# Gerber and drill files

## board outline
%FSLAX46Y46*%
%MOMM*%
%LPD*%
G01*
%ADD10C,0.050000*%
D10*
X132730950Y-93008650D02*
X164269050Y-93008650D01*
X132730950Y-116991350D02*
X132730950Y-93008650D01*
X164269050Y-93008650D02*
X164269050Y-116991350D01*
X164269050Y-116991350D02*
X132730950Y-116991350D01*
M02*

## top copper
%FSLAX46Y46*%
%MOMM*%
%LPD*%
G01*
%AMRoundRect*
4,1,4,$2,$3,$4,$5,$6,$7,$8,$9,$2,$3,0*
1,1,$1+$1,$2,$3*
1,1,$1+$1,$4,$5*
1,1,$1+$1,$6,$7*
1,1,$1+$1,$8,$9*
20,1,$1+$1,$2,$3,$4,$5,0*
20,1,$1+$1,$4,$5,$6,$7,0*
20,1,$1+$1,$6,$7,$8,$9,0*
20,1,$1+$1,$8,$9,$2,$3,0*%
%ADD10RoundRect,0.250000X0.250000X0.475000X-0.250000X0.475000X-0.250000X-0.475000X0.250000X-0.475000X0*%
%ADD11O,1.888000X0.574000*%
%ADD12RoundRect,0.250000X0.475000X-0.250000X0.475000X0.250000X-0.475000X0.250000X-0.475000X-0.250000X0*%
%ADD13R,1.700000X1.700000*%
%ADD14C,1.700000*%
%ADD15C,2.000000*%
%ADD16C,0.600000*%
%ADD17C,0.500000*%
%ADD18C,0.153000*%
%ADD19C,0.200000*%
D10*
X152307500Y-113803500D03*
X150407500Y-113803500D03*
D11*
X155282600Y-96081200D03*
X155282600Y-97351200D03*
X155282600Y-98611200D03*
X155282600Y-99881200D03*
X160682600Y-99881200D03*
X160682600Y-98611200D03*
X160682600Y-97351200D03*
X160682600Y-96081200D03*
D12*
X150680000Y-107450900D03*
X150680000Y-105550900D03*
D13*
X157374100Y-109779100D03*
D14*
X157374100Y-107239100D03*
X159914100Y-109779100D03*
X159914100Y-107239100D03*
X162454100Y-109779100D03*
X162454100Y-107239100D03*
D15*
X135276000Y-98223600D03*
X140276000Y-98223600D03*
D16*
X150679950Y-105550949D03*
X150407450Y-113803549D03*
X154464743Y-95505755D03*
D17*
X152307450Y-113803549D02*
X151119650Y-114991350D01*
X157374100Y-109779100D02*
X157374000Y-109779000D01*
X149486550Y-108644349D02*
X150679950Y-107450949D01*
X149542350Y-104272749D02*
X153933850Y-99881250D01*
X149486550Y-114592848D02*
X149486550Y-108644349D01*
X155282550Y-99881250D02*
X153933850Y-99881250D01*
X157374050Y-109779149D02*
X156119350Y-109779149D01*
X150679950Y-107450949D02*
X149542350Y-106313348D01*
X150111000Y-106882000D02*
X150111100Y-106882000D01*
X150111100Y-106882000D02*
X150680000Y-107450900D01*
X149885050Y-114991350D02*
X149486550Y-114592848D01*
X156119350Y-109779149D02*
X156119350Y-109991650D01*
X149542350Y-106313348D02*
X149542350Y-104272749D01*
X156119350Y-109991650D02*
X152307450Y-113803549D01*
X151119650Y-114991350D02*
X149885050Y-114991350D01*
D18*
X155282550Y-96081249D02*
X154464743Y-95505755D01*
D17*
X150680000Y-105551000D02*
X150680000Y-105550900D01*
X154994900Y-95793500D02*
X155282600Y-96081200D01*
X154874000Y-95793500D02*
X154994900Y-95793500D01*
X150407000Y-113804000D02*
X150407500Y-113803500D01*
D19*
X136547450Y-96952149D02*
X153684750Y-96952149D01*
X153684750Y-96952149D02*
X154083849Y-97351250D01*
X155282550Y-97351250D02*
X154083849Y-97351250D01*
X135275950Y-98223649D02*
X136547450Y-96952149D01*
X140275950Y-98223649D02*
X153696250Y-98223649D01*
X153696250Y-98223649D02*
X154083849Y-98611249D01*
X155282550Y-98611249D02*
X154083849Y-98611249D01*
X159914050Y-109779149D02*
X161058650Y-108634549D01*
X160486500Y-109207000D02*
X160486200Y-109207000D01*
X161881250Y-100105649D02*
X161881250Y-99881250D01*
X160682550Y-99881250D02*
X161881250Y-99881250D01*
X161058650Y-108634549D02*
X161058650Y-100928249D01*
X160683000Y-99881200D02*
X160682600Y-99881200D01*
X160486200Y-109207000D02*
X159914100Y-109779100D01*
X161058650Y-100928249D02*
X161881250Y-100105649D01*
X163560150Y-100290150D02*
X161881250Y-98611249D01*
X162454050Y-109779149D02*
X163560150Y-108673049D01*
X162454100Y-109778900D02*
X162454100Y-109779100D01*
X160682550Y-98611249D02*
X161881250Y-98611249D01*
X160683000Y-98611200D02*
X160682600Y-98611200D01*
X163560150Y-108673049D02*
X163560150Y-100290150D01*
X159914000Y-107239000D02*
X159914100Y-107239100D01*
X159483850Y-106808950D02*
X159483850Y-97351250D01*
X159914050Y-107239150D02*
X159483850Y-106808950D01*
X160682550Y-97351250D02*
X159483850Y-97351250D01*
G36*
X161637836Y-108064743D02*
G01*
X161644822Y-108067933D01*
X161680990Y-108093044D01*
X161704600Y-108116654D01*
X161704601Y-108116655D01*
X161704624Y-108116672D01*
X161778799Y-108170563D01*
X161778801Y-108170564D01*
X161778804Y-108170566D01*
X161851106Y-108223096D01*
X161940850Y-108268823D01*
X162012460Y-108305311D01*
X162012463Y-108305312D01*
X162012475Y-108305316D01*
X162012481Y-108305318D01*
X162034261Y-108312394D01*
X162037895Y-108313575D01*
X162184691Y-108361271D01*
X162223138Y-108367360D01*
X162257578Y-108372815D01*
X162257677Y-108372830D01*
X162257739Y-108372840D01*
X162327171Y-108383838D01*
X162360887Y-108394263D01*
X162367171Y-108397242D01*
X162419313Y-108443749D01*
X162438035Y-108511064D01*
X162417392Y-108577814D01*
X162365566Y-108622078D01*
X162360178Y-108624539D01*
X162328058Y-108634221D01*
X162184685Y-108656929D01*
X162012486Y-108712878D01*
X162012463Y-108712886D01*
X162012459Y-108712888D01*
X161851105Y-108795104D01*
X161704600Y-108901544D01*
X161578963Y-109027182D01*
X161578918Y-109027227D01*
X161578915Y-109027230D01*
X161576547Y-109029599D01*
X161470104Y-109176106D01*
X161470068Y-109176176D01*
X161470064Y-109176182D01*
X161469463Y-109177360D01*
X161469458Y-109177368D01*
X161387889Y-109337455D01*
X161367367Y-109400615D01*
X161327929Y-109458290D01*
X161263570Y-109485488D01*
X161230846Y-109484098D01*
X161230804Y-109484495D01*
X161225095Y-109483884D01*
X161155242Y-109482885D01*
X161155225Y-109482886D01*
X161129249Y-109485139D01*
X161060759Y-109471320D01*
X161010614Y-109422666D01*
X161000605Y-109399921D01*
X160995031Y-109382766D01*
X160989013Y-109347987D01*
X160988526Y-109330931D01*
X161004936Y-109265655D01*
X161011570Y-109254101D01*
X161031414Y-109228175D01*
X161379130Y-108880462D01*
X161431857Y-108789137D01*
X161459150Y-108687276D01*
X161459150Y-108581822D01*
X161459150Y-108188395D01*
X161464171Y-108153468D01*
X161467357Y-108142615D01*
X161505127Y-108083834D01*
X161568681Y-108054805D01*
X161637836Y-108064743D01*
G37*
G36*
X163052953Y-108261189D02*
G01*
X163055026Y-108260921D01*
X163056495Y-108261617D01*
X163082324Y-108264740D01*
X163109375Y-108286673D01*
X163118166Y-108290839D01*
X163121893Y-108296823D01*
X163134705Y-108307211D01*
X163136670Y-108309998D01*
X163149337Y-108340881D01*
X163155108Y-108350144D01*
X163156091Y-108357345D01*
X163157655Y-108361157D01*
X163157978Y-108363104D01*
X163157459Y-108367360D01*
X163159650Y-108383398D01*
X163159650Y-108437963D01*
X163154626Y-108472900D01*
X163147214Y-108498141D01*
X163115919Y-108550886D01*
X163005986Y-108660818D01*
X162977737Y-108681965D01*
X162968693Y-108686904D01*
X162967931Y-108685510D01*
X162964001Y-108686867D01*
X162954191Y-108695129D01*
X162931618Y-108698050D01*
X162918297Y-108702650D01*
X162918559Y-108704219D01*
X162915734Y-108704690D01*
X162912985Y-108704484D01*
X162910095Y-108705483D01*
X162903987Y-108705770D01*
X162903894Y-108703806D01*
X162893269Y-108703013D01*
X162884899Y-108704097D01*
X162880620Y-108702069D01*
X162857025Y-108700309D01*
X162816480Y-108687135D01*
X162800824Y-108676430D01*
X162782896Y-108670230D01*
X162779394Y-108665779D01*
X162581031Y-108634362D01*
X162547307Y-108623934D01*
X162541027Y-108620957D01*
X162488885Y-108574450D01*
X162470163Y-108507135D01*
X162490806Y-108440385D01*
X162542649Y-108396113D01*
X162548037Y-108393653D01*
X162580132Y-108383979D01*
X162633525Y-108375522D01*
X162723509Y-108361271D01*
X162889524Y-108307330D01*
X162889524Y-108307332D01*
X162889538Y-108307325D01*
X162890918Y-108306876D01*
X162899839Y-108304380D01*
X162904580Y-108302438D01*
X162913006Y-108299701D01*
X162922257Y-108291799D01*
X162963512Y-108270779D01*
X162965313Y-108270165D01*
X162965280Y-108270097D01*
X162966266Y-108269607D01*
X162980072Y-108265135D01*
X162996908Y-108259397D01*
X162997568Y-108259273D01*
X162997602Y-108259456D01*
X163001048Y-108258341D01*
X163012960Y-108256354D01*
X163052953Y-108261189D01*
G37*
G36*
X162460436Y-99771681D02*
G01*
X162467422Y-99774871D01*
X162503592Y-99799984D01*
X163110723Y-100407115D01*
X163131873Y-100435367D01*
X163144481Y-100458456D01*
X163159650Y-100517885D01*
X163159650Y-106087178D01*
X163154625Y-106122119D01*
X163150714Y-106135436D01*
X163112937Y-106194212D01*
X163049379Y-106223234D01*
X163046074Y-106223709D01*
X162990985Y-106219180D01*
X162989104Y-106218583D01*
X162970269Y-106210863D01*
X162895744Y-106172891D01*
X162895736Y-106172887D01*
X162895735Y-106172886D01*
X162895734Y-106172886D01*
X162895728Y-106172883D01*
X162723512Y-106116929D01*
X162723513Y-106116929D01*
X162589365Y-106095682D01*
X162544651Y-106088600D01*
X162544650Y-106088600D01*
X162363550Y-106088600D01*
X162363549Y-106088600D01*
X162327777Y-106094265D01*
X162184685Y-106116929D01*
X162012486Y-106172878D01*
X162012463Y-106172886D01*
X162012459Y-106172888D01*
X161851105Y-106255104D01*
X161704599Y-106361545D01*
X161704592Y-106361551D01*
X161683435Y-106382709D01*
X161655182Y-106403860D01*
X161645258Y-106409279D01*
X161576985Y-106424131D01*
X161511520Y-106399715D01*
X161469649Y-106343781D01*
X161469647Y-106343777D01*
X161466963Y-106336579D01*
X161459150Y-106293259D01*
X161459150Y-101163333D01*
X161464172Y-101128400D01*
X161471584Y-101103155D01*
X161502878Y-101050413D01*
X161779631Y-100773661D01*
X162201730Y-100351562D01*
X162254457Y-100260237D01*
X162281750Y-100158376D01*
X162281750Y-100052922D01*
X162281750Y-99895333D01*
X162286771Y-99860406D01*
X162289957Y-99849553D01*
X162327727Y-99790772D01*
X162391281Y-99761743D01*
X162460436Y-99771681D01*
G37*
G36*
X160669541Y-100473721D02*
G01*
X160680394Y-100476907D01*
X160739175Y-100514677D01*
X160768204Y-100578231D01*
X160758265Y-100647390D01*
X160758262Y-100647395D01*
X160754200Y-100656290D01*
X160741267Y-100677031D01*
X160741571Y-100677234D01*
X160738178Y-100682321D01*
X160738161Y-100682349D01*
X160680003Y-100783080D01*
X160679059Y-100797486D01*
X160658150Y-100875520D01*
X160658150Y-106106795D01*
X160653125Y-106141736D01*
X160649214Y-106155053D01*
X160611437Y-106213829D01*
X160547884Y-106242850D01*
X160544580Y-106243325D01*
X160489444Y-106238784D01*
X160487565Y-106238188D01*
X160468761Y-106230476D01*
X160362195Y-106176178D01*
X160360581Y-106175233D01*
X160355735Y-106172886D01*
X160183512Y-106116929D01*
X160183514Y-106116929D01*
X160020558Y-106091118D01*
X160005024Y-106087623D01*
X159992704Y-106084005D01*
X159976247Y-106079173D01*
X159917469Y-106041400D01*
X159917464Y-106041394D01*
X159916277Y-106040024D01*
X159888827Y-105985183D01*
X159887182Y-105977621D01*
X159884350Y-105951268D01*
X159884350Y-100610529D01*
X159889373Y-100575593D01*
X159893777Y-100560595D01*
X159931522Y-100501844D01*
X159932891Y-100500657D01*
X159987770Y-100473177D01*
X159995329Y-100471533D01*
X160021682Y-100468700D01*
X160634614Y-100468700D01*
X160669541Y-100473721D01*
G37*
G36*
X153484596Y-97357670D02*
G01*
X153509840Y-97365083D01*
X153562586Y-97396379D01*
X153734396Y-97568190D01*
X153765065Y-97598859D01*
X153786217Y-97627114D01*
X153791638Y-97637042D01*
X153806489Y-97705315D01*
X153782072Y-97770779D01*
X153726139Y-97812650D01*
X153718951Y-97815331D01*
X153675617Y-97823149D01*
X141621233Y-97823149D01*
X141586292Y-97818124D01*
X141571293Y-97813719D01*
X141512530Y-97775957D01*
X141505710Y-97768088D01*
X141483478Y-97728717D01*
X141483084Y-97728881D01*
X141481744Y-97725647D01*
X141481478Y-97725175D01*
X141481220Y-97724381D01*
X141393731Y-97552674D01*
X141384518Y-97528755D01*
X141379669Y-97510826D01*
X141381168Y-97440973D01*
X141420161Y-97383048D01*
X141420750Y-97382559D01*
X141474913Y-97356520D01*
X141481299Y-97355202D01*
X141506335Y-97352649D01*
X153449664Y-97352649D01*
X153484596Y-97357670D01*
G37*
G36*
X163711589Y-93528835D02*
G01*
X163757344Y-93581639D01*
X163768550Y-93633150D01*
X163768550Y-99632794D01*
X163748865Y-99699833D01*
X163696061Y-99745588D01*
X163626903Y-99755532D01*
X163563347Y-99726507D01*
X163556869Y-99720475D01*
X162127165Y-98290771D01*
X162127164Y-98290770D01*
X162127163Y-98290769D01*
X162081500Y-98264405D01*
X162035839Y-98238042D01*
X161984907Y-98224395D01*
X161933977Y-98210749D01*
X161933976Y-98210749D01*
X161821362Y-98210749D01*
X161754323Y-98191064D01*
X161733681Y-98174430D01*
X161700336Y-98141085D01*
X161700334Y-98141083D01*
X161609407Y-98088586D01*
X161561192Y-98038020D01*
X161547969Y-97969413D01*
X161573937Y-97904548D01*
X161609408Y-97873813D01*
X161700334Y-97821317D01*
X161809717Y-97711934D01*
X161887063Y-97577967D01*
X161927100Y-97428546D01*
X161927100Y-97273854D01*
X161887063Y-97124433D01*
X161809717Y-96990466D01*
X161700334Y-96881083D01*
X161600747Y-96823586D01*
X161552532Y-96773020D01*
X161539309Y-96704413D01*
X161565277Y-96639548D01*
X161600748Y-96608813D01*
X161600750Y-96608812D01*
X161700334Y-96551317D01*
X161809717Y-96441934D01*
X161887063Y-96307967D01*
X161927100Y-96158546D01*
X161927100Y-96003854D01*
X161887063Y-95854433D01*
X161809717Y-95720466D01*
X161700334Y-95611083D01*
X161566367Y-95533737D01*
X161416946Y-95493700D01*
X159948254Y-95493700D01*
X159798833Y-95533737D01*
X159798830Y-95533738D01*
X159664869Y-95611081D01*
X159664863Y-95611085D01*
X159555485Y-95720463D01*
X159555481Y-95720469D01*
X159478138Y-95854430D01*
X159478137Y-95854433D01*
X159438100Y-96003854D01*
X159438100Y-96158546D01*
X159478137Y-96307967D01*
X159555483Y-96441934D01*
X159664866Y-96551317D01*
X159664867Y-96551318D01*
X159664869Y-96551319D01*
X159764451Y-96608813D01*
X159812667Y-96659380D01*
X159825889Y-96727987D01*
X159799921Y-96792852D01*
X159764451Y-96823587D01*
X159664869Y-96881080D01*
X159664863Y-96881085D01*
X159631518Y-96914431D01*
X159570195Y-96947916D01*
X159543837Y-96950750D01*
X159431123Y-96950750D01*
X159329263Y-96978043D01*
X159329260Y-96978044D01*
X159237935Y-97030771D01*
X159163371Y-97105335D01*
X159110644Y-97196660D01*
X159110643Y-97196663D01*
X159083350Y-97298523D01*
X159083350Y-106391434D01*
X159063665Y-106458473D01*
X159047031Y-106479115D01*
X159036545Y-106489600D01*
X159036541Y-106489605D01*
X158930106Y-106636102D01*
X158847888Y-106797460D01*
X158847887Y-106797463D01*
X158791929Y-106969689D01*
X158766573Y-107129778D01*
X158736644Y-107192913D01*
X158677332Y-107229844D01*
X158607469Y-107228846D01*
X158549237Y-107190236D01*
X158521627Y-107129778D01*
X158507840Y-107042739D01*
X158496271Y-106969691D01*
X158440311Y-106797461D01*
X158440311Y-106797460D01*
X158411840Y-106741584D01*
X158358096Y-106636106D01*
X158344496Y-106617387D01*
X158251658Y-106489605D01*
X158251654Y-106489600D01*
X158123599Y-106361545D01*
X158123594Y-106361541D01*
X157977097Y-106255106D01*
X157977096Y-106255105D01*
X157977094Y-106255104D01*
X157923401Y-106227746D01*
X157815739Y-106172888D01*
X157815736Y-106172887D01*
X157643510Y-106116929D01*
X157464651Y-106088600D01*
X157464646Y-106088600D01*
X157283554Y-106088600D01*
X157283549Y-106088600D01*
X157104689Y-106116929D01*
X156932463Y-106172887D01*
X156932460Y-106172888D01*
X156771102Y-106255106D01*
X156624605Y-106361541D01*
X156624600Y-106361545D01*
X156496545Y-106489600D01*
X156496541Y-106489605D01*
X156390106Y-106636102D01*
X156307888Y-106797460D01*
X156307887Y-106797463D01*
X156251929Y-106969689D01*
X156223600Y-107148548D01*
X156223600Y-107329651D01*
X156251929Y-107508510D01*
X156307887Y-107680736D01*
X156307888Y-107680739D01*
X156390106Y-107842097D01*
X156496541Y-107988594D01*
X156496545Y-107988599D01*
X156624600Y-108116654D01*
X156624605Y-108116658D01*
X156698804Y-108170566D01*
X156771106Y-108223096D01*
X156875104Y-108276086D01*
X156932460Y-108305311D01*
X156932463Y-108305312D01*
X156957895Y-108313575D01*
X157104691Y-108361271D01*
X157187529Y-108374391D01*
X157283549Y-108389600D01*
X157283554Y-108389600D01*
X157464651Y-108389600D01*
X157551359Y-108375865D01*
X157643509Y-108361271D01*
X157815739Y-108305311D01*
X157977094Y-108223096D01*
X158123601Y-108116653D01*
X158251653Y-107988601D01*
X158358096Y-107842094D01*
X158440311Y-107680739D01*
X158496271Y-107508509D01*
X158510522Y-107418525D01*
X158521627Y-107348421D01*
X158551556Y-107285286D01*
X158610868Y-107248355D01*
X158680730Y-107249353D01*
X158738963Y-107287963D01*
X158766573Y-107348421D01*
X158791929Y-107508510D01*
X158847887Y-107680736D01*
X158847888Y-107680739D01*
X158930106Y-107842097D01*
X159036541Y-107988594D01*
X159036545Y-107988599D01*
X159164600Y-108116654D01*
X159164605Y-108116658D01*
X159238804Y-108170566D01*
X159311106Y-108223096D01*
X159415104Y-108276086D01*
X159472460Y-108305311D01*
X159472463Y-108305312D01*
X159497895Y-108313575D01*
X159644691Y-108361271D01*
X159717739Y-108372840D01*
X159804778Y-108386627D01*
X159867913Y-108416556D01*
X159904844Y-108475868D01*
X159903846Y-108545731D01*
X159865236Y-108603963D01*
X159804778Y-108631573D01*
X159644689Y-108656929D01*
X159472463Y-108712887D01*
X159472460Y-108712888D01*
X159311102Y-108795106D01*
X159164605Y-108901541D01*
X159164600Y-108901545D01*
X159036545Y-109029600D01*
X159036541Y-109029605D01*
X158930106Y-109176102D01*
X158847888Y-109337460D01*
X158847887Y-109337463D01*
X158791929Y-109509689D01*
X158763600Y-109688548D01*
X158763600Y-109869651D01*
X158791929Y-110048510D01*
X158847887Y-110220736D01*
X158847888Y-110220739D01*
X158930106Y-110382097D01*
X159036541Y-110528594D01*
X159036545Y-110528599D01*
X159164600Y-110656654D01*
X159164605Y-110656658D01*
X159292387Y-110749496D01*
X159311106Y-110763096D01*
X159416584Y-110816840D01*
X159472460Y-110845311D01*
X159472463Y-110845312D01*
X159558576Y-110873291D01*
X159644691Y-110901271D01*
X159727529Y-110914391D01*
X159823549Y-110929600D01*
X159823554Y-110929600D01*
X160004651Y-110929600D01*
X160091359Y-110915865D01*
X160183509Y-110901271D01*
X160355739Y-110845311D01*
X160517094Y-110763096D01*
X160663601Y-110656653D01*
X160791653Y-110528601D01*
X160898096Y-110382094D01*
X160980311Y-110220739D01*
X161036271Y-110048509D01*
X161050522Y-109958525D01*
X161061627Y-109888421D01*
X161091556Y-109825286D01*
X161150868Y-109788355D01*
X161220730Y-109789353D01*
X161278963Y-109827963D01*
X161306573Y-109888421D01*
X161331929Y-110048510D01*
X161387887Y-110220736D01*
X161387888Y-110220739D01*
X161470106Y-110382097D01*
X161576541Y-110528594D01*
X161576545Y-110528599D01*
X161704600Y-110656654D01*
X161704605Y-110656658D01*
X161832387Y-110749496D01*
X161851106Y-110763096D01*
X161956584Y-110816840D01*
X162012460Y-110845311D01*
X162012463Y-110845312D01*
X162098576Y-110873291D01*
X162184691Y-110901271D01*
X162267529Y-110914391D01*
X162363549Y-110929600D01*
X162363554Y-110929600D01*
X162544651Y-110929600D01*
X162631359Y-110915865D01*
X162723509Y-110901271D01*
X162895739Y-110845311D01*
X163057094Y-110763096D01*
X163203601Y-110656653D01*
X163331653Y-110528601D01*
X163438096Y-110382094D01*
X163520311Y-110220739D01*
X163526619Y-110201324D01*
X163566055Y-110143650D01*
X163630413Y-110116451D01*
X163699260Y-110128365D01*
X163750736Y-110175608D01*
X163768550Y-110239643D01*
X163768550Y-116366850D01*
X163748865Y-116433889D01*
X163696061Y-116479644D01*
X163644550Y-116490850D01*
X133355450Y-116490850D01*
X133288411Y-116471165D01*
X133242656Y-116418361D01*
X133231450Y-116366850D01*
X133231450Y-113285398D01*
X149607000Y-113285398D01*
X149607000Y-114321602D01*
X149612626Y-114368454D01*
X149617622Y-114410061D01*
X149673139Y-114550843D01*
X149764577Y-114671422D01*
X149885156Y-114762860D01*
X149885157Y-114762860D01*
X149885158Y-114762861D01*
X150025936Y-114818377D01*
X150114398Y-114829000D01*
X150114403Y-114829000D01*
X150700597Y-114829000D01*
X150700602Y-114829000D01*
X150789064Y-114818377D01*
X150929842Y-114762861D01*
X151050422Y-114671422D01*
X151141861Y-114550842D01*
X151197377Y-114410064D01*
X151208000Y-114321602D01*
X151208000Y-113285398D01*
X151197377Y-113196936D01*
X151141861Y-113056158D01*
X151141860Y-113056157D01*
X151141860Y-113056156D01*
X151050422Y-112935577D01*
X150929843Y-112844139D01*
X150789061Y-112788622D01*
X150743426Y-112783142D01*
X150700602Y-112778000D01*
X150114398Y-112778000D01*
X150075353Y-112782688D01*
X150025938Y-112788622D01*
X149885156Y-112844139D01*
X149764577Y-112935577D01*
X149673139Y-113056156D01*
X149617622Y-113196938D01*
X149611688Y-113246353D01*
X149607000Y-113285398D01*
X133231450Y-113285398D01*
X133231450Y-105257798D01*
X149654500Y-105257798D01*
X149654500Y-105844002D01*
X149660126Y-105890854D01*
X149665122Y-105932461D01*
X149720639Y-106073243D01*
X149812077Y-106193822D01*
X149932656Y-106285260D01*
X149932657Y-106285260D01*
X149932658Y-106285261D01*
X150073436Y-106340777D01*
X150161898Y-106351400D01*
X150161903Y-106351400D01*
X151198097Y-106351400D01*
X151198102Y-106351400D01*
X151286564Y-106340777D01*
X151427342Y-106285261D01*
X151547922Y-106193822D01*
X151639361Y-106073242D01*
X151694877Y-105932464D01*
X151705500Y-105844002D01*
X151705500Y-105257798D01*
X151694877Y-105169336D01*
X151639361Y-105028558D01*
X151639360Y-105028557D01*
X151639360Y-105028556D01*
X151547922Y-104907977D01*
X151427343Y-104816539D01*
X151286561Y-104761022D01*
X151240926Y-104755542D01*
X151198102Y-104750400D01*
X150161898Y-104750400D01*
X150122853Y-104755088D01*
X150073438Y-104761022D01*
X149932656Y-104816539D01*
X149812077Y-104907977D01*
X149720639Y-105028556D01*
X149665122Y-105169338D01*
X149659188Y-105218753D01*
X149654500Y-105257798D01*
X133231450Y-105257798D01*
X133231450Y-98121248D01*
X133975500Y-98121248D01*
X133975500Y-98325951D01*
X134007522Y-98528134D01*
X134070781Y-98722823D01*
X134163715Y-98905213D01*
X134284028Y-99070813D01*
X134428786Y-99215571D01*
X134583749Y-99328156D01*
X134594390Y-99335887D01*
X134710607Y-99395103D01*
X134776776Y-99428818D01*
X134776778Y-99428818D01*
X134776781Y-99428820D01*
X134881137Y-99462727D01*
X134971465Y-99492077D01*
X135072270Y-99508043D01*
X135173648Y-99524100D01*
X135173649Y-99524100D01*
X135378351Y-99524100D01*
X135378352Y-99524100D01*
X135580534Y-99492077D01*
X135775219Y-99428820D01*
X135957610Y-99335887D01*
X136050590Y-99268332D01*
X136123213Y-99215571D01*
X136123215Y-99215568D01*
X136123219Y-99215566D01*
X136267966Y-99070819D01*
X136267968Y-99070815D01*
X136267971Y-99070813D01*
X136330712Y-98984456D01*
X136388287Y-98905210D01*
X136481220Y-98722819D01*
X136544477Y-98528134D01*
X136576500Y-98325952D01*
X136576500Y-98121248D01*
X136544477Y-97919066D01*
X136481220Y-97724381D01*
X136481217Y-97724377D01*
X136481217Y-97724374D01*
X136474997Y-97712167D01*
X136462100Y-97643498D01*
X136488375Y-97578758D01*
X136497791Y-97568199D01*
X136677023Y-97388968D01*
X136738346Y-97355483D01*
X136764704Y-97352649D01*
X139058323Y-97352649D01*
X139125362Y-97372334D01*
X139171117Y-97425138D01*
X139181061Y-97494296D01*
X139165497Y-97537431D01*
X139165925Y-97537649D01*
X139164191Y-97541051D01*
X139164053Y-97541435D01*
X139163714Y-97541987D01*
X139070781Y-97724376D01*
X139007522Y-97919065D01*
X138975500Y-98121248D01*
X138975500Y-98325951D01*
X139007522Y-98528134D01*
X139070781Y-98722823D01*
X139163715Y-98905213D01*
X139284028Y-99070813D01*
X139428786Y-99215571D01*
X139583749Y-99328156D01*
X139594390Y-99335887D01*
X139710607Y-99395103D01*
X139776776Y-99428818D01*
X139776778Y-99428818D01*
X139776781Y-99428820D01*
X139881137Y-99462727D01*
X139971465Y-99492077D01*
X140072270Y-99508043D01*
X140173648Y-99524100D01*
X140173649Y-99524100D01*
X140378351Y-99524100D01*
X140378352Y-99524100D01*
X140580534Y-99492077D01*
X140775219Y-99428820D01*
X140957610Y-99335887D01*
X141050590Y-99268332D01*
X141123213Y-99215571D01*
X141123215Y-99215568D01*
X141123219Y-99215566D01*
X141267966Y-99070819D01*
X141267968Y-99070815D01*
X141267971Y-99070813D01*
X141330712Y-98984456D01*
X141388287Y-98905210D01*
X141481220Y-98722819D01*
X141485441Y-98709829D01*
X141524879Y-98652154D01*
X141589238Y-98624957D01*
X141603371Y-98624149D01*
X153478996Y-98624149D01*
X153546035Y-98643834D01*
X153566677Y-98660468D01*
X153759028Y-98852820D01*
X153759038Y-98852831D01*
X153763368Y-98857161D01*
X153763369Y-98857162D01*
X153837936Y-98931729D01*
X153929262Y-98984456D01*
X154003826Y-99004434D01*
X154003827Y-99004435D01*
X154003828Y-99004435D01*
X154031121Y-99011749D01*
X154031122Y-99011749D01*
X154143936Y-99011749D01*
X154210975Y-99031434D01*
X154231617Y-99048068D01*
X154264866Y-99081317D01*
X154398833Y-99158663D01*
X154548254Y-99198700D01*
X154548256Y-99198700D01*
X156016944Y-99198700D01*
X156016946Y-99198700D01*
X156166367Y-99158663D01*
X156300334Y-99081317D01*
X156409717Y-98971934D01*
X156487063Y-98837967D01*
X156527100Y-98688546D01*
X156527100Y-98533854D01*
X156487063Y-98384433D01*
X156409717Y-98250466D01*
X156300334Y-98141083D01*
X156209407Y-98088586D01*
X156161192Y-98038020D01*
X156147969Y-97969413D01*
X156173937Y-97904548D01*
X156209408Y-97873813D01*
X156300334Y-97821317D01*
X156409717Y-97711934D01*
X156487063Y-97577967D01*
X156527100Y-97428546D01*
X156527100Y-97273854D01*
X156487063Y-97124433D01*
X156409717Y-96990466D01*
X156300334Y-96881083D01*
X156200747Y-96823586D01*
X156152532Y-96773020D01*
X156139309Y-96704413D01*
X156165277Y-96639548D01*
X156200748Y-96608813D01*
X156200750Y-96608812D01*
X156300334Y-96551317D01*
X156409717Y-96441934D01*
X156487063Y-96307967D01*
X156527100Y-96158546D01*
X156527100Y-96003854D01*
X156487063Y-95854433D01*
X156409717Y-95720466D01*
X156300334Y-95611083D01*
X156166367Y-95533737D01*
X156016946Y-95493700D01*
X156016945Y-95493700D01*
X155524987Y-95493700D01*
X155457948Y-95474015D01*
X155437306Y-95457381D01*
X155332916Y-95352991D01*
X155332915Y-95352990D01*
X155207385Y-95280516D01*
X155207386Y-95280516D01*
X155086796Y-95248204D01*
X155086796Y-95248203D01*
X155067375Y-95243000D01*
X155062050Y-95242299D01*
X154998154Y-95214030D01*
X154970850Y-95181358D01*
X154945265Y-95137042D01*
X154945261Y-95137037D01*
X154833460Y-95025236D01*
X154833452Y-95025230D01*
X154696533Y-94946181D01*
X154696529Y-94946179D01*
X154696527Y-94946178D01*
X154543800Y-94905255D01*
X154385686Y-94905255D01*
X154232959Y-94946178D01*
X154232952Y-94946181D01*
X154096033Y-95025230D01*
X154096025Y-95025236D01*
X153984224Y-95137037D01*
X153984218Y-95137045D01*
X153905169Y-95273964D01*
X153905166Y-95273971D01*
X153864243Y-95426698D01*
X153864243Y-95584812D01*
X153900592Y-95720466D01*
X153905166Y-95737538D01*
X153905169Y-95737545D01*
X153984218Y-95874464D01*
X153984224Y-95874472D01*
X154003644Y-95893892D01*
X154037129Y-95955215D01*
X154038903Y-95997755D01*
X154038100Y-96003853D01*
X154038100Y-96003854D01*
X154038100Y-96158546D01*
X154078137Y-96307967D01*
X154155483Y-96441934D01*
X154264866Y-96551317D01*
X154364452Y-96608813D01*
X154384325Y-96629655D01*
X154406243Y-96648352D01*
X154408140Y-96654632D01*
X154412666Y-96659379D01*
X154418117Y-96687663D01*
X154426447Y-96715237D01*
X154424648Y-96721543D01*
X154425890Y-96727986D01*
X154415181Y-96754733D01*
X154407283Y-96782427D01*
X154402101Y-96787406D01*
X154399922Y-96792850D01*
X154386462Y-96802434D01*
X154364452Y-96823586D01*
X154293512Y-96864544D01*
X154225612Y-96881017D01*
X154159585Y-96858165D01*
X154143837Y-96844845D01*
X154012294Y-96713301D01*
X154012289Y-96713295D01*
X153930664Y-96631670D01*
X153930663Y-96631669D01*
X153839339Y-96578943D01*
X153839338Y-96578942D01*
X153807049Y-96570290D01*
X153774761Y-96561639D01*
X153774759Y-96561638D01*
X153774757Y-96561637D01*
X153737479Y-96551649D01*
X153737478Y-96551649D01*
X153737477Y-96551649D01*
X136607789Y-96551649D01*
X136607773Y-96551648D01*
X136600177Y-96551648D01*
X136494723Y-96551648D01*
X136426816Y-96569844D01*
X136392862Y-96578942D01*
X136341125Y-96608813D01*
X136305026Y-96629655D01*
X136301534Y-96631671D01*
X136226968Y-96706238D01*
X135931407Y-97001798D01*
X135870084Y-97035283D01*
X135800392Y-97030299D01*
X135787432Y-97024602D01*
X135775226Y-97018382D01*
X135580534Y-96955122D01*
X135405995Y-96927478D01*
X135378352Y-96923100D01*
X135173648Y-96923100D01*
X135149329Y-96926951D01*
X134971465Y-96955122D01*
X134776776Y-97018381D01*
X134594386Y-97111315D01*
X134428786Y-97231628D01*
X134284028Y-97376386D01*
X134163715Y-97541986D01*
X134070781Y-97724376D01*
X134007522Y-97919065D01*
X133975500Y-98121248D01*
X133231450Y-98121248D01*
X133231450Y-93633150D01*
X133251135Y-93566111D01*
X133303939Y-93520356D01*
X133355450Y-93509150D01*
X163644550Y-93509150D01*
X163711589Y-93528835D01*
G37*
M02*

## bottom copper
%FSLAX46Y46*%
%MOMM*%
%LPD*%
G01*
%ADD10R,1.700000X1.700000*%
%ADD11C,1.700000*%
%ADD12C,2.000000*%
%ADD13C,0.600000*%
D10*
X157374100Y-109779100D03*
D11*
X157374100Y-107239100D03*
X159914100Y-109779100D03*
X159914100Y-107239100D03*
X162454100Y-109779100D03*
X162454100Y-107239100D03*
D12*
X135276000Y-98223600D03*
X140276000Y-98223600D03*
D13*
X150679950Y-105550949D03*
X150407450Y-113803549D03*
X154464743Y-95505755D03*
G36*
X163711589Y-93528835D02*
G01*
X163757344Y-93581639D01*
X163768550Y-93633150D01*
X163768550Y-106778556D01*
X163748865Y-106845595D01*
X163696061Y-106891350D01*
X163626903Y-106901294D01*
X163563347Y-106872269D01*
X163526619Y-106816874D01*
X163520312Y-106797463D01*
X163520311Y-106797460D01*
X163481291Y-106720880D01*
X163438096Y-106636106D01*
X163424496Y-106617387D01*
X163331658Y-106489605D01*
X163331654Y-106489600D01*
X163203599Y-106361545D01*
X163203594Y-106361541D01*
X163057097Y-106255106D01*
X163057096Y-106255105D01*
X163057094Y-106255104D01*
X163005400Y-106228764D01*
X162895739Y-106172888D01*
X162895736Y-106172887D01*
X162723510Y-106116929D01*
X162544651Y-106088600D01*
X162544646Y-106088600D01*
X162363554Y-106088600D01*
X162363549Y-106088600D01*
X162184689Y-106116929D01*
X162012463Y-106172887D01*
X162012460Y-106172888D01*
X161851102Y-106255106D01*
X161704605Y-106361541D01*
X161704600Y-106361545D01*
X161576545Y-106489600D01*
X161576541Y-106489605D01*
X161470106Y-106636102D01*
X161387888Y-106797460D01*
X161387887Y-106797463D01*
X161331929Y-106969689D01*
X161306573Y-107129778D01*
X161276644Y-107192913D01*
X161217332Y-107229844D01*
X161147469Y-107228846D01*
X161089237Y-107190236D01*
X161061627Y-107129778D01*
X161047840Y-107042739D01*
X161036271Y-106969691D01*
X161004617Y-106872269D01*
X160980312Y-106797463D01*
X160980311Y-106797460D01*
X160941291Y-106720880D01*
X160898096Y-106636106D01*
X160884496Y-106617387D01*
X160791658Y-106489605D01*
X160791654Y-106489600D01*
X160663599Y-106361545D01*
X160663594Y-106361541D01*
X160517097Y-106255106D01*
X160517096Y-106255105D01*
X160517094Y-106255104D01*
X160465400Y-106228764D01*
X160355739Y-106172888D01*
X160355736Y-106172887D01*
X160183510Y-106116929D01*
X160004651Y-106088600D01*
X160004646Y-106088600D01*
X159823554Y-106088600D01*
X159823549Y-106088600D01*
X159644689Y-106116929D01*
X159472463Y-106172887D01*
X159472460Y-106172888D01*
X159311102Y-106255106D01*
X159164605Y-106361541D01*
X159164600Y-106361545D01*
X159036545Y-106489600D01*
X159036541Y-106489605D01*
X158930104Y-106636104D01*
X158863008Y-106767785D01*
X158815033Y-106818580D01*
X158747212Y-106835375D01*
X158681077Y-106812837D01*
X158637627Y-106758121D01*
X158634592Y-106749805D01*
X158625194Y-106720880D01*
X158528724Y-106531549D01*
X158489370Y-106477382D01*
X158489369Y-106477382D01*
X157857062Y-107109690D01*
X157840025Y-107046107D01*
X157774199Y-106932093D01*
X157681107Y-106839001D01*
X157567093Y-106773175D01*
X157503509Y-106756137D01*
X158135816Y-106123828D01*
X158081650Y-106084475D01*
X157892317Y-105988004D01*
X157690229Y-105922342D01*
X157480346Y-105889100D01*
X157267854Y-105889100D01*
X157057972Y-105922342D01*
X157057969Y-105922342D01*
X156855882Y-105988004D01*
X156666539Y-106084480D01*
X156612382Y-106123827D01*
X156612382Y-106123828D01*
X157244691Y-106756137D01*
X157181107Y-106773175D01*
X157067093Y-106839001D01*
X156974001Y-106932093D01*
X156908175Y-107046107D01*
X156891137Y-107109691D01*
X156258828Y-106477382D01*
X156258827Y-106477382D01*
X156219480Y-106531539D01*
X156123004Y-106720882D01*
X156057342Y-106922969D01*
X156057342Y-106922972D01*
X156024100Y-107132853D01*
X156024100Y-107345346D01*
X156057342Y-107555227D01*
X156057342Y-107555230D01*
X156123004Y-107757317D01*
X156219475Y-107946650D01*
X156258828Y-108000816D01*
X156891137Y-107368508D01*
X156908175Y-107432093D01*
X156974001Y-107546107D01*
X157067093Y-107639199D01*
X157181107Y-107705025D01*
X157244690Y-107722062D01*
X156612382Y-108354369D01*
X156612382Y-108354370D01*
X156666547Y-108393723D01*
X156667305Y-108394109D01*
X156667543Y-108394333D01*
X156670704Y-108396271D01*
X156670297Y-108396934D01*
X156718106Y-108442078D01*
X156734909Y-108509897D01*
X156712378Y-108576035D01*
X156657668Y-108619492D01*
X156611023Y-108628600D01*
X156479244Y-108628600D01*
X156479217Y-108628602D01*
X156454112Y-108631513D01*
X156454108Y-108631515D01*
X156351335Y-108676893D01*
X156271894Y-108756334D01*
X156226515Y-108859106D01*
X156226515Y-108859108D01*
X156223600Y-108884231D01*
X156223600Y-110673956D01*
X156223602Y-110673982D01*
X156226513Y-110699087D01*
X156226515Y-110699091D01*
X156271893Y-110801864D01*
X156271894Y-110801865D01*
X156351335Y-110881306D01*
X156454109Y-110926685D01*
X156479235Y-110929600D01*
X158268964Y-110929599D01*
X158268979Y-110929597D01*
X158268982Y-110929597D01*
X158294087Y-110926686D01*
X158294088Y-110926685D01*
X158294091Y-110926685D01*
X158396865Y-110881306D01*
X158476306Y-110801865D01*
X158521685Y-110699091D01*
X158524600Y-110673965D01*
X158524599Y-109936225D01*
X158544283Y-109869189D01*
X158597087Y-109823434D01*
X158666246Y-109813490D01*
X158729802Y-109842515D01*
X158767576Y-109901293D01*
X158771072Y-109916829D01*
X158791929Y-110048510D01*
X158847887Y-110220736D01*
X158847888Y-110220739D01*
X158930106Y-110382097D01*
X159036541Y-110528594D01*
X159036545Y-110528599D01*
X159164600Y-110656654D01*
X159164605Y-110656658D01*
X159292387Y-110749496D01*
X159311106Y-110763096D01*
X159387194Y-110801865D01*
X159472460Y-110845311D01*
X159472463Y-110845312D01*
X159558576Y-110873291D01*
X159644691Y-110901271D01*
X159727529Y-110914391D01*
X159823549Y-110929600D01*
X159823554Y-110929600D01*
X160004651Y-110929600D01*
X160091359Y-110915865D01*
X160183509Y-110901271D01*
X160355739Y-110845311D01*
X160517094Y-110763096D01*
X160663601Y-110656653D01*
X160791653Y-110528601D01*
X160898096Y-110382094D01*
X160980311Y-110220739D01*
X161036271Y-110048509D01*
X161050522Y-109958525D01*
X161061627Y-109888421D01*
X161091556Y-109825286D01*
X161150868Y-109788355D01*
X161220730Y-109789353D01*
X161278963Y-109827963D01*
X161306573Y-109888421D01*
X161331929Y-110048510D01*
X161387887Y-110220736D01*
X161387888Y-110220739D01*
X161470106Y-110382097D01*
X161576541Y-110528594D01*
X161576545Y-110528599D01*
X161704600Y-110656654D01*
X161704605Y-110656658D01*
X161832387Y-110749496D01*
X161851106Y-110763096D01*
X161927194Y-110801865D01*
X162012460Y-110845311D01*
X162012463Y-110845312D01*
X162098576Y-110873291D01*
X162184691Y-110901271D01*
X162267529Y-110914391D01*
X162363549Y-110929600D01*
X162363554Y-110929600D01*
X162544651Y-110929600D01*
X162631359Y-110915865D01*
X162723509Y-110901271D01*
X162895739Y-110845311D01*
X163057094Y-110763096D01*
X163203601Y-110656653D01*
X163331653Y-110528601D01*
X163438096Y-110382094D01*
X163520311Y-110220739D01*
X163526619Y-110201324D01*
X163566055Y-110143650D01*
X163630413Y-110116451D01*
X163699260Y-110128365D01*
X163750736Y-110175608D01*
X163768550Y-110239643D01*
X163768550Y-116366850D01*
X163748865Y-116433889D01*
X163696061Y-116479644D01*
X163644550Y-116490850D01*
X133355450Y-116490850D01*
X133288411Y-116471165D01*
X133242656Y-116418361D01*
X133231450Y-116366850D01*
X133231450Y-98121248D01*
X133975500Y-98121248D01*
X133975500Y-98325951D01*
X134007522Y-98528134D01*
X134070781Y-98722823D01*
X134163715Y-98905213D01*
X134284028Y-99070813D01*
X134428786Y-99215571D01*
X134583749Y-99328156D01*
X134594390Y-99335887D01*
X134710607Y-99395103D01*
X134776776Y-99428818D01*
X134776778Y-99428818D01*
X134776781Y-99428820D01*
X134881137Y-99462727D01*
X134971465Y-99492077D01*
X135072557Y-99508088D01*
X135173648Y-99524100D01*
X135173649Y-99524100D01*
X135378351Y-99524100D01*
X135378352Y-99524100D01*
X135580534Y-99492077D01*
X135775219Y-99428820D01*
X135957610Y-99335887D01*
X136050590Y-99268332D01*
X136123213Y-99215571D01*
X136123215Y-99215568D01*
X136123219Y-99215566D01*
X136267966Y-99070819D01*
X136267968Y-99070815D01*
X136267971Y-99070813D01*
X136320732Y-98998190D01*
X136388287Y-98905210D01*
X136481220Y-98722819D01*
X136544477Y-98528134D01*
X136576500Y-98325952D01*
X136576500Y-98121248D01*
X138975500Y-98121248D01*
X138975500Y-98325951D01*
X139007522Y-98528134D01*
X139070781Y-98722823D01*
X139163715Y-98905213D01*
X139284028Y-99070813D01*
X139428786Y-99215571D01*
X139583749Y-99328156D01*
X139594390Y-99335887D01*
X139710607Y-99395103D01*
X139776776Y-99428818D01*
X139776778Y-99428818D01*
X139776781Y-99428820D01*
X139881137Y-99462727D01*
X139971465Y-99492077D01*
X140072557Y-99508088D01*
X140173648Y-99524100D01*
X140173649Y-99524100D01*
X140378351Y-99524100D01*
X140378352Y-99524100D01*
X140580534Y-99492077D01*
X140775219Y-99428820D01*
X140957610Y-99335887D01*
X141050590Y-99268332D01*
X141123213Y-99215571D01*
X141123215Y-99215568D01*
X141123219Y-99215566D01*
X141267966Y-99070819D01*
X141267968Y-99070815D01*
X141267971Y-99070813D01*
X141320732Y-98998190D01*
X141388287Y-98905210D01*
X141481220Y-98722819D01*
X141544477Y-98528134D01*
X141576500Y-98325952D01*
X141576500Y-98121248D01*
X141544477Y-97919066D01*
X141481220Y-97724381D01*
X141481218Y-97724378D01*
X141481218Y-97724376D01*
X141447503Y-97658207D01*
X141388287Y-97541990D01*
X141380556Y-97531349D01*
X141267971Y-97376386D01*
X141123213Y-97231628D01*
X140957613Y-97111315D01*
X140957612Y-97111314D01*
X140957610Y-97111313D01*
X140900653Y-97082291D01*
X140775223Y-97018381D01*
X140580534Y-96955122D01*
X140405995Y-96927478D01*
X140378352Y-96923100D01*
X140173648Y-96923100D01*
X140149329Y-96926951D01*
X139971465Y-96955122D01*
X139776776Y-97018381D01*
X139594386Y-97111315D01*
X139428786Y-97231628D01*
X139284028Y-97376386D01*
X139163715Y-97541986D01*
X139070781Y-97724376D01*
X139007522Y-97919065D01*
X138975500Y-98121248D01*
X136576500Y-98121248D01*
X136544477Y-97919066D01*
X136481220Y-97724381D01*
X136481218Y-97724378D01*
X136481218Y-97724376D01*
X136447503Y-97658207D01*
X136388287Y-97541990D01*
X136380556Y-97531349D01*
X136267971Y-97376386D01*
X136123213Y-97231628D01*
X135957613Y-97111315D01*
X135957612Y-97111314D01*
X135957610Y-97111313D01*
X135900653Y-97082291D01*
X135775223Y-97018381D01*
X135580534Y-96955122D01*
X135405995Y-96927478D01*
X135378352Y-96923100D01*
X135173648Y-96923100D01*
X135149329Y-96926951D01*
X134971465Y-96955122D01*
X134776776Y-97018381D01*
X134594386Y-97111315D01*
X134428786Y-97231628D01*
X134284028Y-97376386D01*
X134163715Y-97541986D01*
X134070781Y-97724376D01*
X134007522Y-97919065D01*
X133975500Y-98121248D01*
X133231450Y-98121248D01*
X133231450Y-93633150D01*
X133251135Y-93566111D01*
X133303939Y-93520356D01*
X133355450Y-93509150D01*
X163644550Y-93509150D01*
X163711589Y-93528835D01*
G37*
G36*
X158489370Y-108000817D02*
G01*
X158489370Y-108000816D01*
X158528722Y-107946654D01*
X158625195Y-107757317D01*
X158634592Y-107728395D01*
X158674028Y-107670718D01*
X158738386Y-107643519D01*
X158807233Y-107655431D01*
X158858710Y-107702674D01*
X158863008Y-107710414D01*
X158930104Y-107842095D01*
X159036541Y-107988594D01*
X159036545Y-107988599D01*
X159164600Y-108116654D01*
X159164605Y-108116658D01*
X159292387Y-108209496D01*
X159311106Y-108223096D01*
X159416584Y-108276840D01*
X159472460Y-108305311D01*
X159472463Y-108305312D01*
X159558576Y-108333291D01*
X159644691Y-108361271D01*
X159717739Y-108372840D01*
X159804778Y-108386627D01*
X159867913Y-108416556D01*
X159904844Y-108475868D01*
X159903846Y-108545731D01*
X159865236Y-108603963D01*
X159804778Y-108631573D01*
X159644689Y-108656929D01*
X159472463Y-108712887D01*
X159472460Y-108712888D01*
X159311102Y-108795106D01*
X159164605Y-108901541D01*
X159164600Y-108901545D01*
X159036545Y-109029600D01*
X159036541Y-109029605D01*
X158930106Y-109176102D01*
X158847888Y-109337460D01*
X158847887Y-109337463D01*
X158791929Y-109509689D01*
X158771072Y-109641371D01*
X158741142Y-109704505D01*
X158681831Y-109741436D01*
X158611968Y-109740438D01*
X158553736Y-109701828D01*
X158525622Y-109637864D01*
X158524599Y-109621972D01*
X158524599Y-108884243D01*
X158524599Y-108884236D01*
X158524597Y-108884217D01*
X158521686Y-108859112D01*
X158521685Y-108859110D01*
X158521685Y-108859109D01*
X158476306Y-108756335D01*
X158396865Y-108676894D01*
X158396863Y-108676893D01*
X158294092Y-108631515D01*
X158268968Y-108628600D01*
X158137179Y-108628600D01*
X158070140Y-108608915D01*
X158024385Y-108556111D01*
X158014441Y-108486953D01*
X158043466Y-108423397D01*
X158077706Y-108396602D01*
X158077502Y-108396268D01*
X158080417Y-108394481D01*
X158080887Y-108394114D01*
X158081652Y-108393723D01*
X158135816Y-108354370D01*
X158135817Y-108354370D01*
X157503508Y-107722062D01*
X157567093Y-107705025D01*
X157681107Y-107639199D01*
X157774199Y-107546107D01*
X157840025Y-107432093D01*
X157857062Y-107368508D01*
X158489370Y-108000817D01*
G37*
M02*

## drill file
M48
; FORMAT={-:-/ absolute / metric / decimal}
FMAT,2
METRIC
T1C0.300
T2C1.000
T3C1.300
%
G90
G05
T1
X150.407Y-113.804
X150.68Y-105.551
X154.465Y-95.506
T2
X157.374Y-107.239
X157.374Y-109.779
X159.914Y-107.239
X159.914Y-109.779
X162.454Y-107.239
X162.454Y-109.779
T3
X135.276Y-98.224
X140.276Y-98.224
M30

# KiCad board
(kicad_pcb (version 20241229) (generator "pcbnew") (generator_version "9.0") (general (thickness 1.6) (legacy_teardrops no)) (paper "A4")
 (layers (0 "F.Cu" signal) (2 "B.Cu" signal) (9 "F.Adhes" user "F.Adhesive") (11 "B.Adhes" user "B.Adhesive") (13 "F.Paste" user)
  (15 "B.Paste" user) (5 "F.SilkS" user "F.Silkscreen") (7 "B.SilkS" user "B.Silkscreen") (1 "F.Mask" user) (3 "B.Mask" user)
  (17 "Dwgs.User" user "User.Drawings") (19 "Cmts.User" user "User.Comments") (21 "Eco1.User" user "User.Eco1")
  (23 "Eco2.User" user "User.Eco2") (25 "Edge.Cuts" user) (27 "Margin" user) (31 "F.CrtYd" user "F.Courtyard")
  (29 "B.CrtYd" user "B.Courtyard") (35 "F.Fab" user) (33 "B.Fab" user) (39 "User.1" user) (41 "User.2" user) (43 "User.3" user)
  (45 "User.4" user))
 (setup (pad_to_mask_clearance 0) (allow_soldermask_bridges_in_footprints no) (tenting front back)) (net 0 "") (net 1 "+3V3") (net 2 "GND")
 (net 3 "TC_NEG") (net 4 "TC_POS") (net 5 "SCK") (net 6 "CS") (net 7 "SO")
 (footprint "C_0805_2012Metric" (layer "F.Cu") (at 151.3575 113.8035 180)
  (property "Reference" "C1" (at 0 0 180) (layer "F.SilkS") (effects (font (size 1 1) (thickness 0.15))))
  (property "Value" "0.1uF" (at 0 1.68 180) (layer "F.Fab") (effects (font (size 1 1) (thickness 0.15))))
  (pad "1" smd roundrect (at -0.95 0 180) (size 1 1.45) (layers "F.Cu" "F.Mask" "F.Paste") (roundrect_rratio 0.25) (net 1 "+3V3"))
  (pad "2" smd roundrect (at 0.95 0 180) (size 1 1.45) (layers "F.Cu" "F.Mask" "F.Paste") (roundrect_rratio 0.25) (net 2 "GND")))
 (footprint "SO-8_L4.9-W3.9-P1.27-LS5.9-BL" (layer "F.Cu") (at 157.9826 97.9812 -90)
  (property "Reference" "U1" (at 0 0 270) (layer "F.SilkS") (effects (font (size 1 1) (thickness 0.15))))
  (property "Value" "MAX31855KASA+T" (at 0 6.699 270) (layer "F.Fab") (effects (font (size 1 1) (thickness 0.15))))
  (pad "1" smd oval (at -1.9 2.7 270) (size 0.574 1.888) (layers "F.Cu" "F.Mask" "F.Paste") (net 2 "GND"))
  (pad "2" smd oval (at -0.63 2.7 270) (size 0.574 1.888) (layers "F.Cu" "F.Mask" "F.Paste") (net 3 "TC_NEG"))
  (pad "3" smd oval (at 0.63 2.7 270) (size 0.574 1.888) (layers "F.Cu" "F.Mask" "F.Paste") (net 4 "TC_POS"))
  (pad "4" smd oval (at 1.9 2.7 270) (size 0.574 1.888) (layers "F.Cu" "F.Mask" "F.Paste") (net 1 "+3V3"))
  (pad "5" smd oval (at 1.9 -2.7 270) (size 0.574 1.888) (layers "F.Cu" "F.Mask" "F.Paste") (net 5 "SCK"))
  (pad "6" smd oval (at 0.63 -2.7 270) (size 0.574 1.888) (layers "F.Cu" "F.Mask" "F.Paste") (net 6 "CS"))
  (pad "7" smd oval (at -0.63 -2.7 270) (size 0.574 1.888) (layers "F.Cu" "F.Mask" "F.Paste") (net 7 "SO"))
  (pad "8" smd oval (at -1.9 -2.7 270) (size 0.574 1.888) (layers "F.Cu" "F.Mask" "F.Paste")))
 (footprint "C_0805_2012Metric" (layer "F.Cu") (at 150.68 106.5009 90)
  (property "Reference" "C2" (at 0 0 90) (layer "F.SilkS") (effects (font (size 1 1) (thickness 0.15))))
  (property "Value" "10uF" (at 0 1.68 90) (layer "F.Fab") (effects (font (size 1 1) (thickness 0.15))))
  (pad "1" smd roundrect (at -0.95 0 90) (size 1 1.45) (layers "F.Cu" "F.Mask" "F.Paste") (roundrect_rratio 0.25) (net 1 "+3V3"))
  (pad "2" smd roundrect (at 0.95 0 90) (size 1 1.45) (layers "F.Cu" "F.Mask" "F.Paste") (roundrect_rratio 0.25) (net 2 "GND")))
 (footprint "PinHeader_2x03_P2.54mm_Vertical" (layer "F.Cu") (at 157.3741 109.7791 90)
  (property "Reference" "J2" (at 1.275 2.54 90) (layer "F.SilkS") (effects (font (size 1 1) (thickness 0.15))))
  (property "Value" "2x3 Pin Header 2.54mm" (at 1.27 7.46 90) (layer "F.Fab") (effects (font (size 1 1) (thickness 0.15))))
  (pad "1" thru_hole rect (at 0 0 90) (size 1.7 1.7) (drill 1) (layers "*.Cu" "*.Mask") (remove_unused_layers no) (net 1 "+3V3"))
  (pad "2" thru_hole circle (at 2.54 0 90) (size 1.7 1.7) (drill 1) (layers "*.Cu" "*.Mask") (remove_unused_layers no) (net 2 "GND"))
  (pad "3" thru_hole circle (at 0 2.54 90) (size 1.7 1.7) (drill 1) (layers "*.Cu" "*.Mask") (remove_unused_layers no) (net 5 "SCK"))
  (pad "4" thru_hole circle (at 2.54 2.54 90) (size 1.7 1.7) (drill 1) (layers "*.Cu" "*.Mask") (remove_unused_layers no) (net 7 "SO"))
  (pad "5" thru_hole circle (at 0 5.08 90) (size 1.7 1.7) (drill 1) (layers "*.Cu" "*.Mask") (remove_unused_layers no) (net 6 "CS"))
  (pad "6" thru_hole circle (at 2.54 5.08 90) (size 1.7 1.7) (drill 1) (layers "*.Cu" "*.Mask") (remove_unused_layers no)))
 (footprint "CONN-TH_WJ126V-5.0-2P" (layer "F.Cu") (at 137.776 98.2236 90)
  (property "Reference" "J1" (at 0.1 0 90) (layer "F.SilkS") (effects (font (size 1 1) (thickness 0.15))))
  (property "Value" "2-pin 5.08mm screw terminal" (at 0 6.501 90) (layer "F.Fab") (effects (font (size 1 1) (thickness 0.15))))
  (pad "1" thru_hole circle (at 0 -2.5 90) (size 2 2) (drill 1.300022) (layers "*.Cu" "*.Mask") (remove_unused_layers no) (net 3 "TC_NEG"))
  (pad "2" thru_hole circle (at 0 2.5 90) (size 2 2) (drill 1.300022) (layers "*.Cu" "*.Mask") (remove_unused_layers no) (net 4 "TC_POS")))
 (gr_line (start 132.73095 93.00865) (end 164.26905 93.00865) (stroke (width 0.05) (type default)) (layer "Edge.Cuts"))
 (gr_line (start 132.73095 116.99135) (end 132.73095 93.00865) (stroke (width 0.05) (type default)) (layer "Edge.Cuts"))
 (gr_line (start 164.26905 93.00865) (end 164.26905 116.99135) (stroke (width 0.05) (type default)) (layer "Edge.Cuts"))
 (gr_line (start 164.26905 116.99135) (end 132.73095 116.99135) (stroke (width 0.05) (type default)) (layer "Edge.Cuts"))
 (segment (start 152.30745 113.803549) (end 151.11965 114.99135) (width 0.5) (layer "F.Cu") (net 1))
 (segment (start 157.3741 109.7791) (end 157.374 109.779) (width 0.5) (layer "F.Cu") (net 1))
 (segment (start 149.48655 108.644349) (end 150.67995 107.450949) (width 0.5) (layer "F.Cu") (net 1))
 (segment (start 149.54235 104.272749) (end 153.93385 99.88125) (width 0.5) (layer "F.Cu") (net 1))
 (segment (start 149.48655 114.592848) (end 149.48655 108.644349) (width 0.5) (layer "F.Cu") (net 1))
 (segment (start 155.28255 99.88125) (end 153.93385 99.88125) (width 0.5) (layer "F.Cu") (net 1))
 (segment (start 157.37405 109.779149) (end 156.11935 109.779149) (width 0.5) (layer "F.Cu") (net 1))
 (segment (start 150.67995 107.450949) (end 149.54235 106.313348) (width 0.5) (layer "F.Cu") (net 1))
 (segment (start 150.111 106.882) (end 150.1111 106.882) (width 0.5) (layer "F.Cu") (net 1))
 (segment (start 150.1111 106.882) (end 150.68 107.4509) (width 0.5) (layer "F.Cu") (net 1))
 (segment (start 149.88505 114.99135) (end 149.48655 114.592848) (width 0.5) (layer "F.Cu") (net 1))
 (segment (start 156.11935 109.779149) (end 156.11935 109.99165) (width 0.5) (layer "F.Cu") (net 1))
 (segment (start 149.54235 106.313348) (end 149.54235 104.272749) (width 0.5) (layer "F.Cu") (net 1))
 (segment (start 156.11935 109.99165) (end 152.30745 113.803549) (width 0.5) (layer "F.Cu") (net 1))
 (segment (start 151.11965 114.99135) (end 149.88505 114.99135) (width 0.5) (layer "F.Cu") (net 1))
 (segment (start 155.28255 96.081249) (end 154.464743 95.505755) (width 0.153) (layer "F.Cu") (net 2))
 (segment (start 150.68 105.551) (end 150.68 105.5509) (width 0.5) (layer "F.Cu") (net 2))
 (segment (start 154.9949 95.7935) (end 155.2826 96.0812) (width 0.5) (layer "F.Cu") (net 2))
 (segment (start 154.874 95.7935) (end 154.9949 95.7935) (width 0.5) (layer "F.Cu") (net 2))
 (segment (start 150.407 113.804) (end 150.4075 113.8035) (width 0.5) (layer "F.Cu") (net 2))
 (via (at 150.67995 105.550949) (size 0.6) (drill 0.3) (layers "F.Cu" "B.Cu") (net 2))
 (via (at 150.40745 113.803549) (size 0.6) (drill 0.3) (layers "F.Cu" "B.Cu") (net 2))
 (via (at 154.464743 95.505755) (size 0.6) (drill 0.3) (layers "F.Cu" "B.Cu") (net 2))
 (segment (start 136.54745 96.952149) (end 153.68475 96.952149) (width 0.2) (layer "F.Cu") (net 3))
 (segment (start 153.68475 96.952149) (end 154.083849 97.35125) (width 0.2) (layer "F.Cu") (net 3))
 (segment (start 155.28255 97.35125) (end 154.083849 97.35125) (width 0.2) (layer "F.Cu") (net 3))
 (segment (start 135.27595 98.223649) (end 136.54745 96.952149) (width 0.2) (layer "F.Cu") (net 3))
 (segment (start 140.27595 98.223649) (end 153.69625 98.223649) (width 0.2) (layer "F.Cu") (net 4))
 (segment (start 153.69625 98.223649) (end 154.083849 98.611249) (width 0.2) (layer "F.Cu") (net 4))
 (segment (start 155.28255 98.611249) (end 154.083849 98.611249) (width 0.2) (layer "F.Cu") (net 4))
 (segment (start 159.91405 109.779149) (end 161.05865 108.634549) (width 0.2) (layer "F.Cu") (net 5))
 (segment (start 160.4865 109.207) (end 160.4862 109.207) (width 0.2) (layer "F.Cu") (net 5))
 (segment (start 161.88125 100.105649) (end 161.88125 99.88125) (width 0.2) (layer "F.Cu") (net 5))
 (segment (start 160.68255 99.88125) (end 161.88125 99.88125) (width 0.2) (layer "F.Cu") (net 5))
 (segment (start 161.05865 108.634549) (end 161.05865 100.928249) (width 0.2) (layer "F.Cu") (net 5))
 (segment (start 160.683 99.8812) (end 160.6826 99.8812) (width 0.2) (layer "F.Cu") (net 5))
 (segment (start 160.4862 109.207) (end 159.9141 109.7791) (width 0.2) (layer "F.Cu") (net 5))
 (segment (start 161.05865 100.928249) (end 161.88125 100.105649) (width 0.2) (layer "F.Cu") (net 5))
 (segment (start 163.56015 100.29015) (end 161.88125 98.611249) (width 0.2) (layer "F.Cu") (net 6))
 (segment (start 162.45405 109.779149) (end 163.56015 108.673049) (width 0.2) (layer "F.Cu") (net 6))
 (segment (start 162.4541 109.7789) (end 162.4541 109.7791) (width 0.2) (layer "F.Cu") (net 6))
 (segment (start 160.68255 98.611249) (end 161.88125 98.611249) (width 0.2) (layer "F.Cu") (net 6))
 (segment (start 160.683 98.6112) (end 160.6826 98.6112) (width 0.2) (layer "F.Cu") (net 6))
 (segment (start 163.56015 108.673049) (end 163.56015 100.29015) (width 0.2) (layer "F.Cu") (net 6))
 (segment (start 159.914 107.239) (end 159.9141 107.2391) (width 0.2) (layer "F.Cu") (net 7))
 (segment (start 159.48385 106.80895) (end 159.48385 97.35125) (width 0.2) (layer "F.Cu") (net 7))
 (segment (start 159.91405 107.23915) (end 159.48385 106.80895) (width 0.2) (layer "F.Cu") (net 7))
 (segment (start 160.68255 97.35125) (end 159.48385 97.35125) (width 0.2) (layer "F.Cu") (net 7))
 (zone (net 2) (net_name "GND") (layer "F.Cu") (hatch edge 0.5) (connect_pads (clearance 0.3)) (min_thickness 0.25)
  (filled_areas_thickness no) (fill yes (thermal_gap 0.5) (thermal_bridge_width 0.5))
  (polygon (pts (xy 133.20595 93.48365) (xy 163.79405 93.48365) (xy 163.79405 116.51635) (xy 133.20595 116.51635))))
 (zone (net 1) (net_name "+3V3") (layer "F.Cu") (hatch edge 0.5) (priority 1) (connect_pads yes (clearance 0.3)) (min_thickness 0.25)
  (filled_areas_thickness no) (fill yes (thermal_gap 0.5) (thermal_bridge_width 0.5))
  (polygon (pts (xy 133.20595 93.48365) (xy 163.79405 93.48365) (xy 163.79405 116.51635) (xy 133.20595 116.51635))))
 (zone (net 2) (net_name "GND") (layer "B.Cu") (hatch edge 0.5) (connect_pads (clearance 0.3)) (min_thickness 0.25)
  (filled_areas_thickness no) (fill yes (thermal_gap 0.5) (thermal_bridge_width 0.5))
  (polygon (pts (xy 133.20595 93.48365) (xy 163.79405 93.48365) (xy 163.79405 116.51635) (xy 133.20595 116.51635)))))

